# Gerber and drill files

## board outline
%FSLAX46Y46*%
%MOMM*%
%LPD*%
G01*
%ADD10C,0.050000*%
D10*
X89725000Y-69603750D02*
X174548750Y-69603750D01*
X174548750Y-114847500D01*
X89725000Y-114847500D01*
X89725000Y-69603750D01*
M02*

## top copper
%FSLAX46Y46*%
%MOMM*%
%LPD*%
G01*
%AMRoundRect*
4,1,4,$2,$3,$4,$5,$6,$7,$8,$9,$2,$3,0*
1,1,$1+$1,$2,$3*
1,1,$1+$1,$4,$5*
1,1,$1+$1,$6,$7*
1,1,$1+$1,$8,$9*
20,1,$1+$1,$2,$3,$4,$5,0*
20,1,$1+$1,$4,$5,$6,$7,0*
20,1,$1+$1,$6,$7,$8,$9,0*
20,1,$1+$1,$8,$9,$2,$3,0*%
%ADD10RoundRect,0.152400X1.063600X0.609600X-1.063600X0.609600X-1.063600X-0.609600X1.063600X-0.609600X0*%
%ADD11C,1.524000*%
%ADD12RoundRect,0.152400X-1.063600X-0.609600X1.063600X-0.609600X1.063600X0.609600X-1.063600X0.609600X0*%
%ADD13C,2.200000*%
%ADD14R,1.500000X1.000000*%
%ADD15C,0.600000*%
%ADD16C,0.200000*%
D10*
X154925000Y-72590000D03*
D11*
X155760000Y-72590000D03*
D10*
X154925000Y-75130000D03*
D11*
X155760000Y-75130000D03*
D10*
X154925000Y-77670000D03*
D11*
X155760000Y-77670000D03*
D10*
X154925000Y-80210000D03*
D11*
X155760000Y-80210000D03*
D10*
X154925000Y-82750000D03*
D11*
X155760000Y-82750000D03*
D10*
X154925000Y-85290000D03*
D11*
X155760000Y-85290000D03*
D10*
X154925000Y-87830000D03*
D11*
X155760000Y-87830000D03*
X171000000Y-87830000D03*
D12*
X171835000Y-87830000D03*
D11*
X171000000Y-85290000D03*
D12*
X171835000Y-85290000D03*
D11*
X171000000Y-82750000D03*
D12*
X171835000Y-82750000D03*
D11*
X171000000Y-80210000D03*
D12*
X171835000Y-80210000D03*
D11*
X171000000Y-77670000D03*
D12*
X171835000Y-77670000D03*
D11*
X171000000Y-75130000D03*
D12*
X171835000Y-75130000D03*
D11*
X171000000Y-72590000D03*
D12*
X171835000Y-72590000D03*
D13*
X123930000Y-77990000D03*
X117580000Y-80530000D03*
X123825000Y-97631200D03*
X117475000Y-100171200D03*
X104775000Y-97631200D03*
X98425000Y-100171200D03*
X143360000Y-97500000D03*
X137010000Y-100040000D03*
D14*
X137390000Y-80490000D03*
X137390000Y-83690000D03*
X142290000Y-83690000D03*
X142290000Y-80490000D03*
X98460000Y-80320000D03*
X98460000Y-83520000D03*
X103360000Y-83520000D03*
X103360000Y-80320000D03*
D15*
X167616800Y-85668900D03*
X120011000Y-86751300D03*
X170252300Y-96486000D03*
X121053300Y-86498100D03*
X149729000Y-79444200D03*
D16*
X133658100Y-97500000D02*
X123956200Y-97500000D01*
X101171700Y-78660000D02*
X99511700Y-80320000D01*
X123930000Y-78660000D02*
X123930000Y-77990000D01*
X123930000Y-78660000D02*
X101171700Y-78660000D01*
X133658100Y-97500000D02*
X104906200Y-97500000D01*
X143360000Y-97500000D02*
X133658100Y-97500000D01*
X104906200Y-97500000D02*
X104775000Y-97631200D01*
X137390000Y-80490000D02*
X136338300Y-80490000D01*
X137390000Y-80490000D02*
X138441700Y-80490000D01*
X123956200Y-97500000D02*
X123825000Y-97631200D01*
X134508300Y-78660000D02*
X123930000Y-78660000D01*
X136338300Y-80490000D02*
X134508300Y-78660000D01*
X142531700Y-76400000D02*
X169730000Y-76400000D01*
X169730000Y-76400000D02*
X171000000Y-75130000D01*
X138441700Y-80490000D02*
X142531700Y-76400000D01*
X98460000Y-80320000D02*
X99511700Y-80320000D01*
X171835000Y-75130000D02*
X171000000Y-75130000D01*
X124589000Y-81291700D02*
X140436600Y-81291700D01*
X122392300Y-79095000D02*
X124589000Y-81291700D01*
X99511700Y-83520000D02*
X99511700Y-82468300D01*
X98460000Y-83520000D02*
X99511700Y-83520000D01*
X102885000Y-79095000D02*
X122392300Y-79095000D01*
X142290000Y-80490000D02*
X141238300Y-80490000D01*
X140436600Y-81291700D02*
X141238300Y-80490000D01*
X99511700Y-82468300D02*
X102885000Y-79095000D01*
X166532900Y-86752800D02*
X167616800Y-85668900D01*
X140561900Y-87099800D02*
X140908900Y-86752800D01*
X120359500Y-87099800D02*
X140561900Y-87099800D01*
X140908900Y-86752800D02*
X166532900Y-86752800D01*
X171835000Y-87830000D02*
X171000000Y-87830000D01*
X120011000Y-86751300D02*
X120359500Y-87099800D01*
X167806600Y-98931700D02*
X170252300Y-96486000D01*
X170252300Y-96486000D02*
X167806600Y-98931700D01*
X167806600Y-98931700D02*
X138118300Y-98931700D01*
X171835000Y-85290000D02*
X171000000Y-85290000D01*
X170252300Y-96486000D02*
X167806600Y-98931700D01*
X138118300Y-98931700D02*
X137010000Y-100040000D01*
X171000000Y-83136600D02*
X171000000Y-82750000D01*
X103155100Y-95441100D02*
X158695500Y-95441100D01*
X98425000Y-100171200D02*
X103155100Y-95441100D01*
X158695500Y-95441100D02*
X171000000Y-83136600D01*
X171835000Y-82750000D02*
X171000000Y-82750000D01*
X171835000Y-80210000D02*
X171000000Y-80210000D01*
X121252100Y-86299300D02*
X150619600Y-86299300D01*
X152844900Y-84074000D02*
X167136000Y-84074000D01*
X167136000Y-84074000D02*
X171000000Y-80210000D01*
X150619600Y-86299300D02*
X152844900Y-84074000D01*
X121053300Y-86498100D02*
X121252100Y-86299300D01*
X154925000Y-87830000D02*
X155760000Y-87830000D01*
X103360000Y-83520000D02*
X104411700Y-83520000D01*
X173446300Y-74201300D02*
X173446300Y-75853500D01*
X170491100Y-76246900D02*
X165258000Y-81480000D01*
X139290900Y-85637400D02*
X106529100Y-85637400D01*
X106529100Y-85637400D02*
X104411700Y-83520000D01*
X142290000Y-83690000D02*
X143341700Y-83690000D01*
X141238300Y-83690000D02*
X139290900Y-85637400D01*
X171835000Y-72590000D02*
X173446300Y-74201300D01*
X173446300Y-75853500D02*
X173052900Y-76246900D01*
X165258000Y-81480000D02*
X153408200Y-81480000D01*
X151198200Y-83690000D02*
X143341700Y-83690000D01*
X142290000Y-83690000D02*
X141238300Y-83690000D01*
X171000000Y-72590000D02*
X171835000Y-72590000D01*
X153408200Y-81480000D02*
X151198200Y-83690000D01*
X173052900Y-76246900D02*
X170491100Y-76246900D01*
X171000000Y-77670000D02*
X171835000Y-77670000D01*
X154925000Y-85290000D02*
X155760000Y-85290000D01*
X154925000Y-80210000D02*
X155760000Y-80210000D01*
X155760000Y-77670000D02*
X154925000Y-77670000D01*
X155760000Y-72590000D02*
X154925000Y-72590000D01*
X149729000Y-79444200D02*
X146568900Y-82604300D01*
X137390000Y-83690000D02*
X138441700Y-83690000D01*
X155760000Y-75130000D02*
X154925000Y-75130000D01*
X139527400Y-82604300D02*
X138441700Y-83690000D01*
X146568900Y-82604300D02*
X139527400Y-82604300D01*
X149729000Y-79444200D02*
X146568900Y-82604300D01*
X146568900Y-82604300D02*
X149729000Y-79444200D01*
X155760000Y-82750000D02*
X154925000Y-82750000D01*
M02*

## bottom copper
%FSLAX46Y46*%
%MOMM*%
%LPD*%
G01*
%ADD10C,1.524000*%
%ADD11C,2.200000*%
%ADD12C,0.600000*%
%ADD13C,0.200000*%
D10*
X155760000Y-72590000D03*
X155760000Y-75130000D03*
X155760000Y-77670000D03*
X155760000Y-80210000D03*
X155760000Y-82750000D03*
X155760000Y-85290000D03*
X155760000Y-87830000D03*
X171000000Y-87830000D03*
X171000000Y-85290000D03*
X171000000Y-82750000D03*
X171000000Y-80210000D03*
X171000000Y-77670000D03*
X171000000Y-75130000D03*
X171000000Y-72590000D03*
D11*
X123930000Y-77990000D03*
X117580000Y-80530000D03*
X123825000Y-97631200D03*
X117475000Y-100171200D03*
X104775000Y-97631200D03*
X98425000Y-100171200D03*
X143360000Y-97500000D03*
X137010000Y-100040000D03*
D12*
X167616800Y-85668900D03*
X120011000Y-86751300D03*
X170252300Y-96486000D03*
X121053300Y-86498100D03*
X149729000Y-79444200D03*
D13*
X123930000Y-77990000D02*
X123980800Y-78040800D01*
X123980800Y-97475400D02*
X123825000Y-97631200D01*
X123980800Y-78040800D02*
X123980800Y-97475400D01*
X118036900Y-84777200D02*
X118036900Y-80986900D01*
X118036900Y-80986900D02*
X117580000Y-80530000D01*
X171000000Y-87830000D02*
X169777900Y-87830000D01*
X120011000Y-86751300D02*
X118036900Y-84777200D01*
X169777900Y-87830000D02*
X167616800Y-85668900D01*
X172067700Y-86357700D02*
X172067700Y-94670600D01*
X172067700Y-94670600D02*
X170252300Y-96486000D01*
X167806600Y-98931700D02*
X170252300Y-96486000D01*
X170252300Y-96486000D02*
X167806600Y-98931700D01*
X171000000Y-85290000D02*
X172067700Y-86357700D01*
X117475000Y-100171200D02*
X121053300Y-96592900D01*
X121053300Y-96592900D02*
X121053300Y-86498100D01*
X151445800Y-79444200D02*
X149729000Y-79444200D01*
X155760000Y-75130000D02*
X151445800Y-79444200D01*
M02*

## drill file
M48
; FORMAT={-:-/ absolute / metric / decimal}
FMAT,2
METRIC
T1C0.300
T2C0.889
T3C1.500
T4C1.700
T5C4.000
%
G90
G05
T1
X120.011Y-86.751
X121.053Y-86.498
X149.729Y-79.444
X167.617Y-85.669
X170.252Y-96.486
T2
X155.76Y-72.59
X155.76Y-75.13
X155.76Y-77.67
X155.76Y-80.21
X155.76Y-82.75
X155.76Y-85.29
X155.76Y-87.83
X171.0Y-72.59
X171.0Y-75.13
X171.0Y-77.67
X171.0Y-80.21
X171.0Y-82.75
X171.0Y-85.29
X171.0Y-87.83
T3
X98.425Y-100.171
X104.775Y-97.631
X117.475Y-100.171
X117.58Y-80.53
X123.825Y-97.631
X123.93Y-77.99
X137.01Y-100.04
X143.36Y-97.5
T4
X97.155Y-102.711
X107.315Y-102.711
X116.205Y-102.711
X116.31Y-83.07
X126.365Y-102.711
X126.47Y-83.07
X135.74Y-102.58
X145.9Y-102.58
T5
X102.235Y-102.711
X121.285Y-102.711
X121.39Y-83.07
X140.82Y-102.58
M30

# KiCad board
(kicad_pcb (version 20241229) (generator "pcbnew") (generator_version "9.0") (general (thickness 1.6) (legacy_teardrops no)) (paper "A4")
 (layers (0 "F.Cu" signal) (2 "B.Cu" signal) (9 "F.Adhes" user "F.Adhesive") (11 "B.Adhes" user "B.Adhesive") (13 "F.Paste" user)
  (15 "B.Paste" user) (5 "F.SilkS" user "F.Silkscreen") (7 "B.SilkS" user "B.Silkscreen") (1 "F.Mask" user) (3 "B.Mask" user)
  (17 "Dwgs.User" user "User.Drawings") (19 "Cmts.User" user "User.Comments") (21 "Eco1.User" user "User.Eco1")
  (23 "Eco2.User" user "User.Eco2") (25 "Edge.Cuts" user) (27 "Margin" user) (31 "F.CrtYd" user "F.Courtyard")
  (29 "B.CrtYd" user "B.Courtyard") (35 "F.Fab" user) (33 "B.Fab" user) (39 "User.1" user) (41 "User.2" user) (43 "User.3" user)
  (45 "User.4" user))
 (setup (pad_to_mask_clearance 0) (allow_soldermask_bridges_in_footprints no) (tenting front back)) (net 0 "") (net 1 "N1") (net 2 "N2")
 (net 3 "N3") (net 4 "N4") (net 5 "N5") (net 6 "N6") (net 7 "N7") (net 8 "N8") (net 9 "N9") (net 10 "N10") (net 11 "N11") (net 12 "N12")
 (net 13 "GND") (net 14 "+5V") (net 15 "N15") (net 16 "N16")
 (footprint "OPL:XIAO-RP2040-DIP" (layer "F.Cu") (at 163.38 80.21)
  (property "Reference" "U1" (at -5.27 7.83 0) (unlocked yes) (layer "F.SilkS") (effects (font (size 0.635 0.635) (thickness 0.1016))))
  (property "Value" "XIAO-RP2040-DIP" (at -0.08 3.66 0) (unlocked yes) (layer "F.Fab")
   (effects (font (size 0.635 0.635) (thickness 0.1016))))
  (pad "1" smd roundrect (at -8.455 -7.62 180) (size 2.432 1.524) (layers "F.Cu" "F.Mask") (roundrect_rratio 0.1) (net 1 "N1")
   (thermal_bridge_angle 45))
  (pad "1" thru_hole circle (at -7.62 -7.62 180) (size 1.524 1.524) (drill 0.889) (layers "*.Cu" "*.Mask") (remove_unused_layers no)
   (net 1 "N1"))
  (pad "2" smd roundrect (at -8.455 -5.08 180) (size 2.432 1.524) (layers "F.Cu" "F.Mask") (roundrect_rratio 0.1) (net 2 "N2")
   (thermal_bridge_angle 45))
  (pad "2" thru_hole circle (at -7.62 -5.08 180) (size 1.524 1.524) (drill 0.889) (layers "*.Cu" "*.Mask") (remove_unused_layers no)
   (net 2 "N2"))
  (pad "3" smd roundrect (at -8.455 -2.54 180) (size 2.432 1.524) (layers "F.Cu" "F.Mask") (roundrect_rratio 0.1) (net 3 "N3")
   (thermal_bridge_angle 45))
  (pad "3" thru_hole circle (at -7.62 -2.54 180) (size 1.524 1.524) (drill 0.889) (layers "*.Cu" "*.Mask") (remove_unused_layers no)
   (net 3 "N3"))
  (pad "4" smd roundrect (at -8.455 0 180) (size 2.432 1.524) (layers "F.Cu" "F.Mask") (roundrect_rratio 0.1) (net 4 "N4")
   (thermal_bridge_angle 45))
  (pad "4" thru_hole circle (at -7.62 0 180) (size 1.524 1.524) (drill 0.889) (layers "*.Cu" "*.Mask") (remove_unused_layers no)
   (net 4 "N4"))
  (pad "5" smd roundrect (at -8.455 2.54 180) (size 2.432 1.524) (layers "F.Cu" "F.Mask") (roundrect_rratio 0.1) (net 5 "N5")
   (thermal_bridge_angle 45))
  (pad "5" thru_hole circle (at -7.62 2.54 180) (size 1.524 1.524) (drill 0.889) (layers "*.Cu" "*.Mask") (remove_unused_layers no)
   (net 5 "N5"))
  (pad "6" smd roundrect (at -8.455 5.08 180) (size 2.432 1.524) (layers "F.Cu" "F.Mask") (roundrect_rratio 0.1) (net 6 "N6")
   (thermal_bridge_angle 45))
  (pad "6" thru_hole circle (at -7.62 5.08 180) (size 1.524 1.524) (drill 0.889) (layers "*.Cu" "*.Mask") (remove_unused_layers no)
   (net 6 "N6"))
  (pad "7" smd roundrect (at -8.455 7.62 180) (size 2.432 1.524) (layers "F.Cu" "F.Mask") (roundrect_rratio 0.1) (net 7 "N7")
   (thermal_bridge_angle 45))
  (pad "7" thru_hole circle (at -7.62 7.62 180) (size 1.524 1.524) (drill 0.889) (layers "*.Cu" "*.Mask") (remove_unused_layers no)
   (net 7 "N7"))
  (pad "8" thru_hole circle (at 7.62 7.62) (size 1.524 1.524) (drill 0.889) (layers "*.Cu" "*.Mask") (remove_unused_layers no) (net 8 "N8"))
  (pad "8" smd roundrect (at 8.455 7.62) (size 2.432 1.524) (layers "F.Cu" "F.Mask") (roundrect_rratio 0.1) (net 8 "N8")
   (thermal_bridge_angle 45))
  (pad "9" thru_hole circle (at 7.62 5.08) (size 1.524 1.524) (drill 0.889) (layers "*.Cu" "*.Mask") (remove_unused_layers no) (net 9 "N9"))
  (pad "9" smd roundrect (at 8.455 5.08) (size 2.432 1.524) (layers "F.Cu" "F.Mask") (roundrect_rratio 0.1) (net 9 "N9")
   (thermal_bridge_angle 45))
  (pad "10" thru_hole circle (at 7.62 2.54) (size 1.524 1.524) (drill 0.889) (layers "*.Cu" "*.Mask") (remove_unused_layers no)
   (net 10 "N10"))
  (pad "10" smd roundrect (at 8.455 2.54) (size 2.432 1.524) (layers "F.Cu" "F.Mask") (roundrect_rratio 0.1) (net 10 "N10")
   (thermal_bridge_angle 45))
  (pad "11" thru_hole circle (at 7.62 0) (size 1.524 1.524) (drill 0.889) (layers "*.Cu" "*.Mask") (remove_unused_layers no) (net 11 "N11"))
  (pad "11" smd roundrect (at 8.455 0) (size 2.432 1.524) (layers "F.Cu" "F.Mask") (roundrect_rratio 0.1) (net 11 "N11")
   (thermal_bridge_angle 45))
  (pad "12" thru_hole circle (at 7.62 -2.54) (size 1.524 1.524) (drill 0.889) (layers "*.Cu" "*.Mask") (remove_unused_layers no)
   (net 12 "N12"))
  (pad "12" smd roundrect (at 8.455 -2.54) (size 2.432 1.524) (layers "F.Cu" "F.Mask") (roundrect_rratio 0.1) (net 12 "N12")
   (thermal_bridge_angle 45))
  (pad "13" thru_hole circle (at 7.62 -5.08) (size 1.524 1.524) (drill 0.889) (layers "*.Cu" "*.Mask") (remove_unused_layers no)
   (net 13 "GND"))
  (pad "13" smd roundrect (at 8.455 -5.08) (size 2.432 1.524) (layers "F.Cu" "F.Mask") (roundrect_rratio 0.1) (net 13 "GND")
   (thermal_bridge_angle 45))
  (pad "14" thru_hole circle (at 7.62 -7.62) (size 1.524 1.524) (drill 0.889) (layers "*.Cu" "*.Mask") (remove_unused_layers no)
   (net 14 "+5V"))
  (pad "14" smd roundrect (at 8.455 -7.62) (size 2.432 1.524) (layers "F.Cu" "F.Mask") (roundrect_rratio 0.1) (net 14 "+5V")
   (thermal_bridge_angle 45)))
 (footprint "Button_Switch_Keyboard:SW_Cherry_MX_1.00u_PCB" (layer "F.Cu") (at 123.93 77.99)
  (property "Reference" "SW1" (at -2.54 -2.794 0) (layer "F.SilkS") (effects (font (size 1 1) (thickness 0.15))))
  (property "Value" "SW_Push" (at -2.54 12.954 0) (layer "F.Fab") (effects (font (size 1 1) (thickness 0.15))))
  (pad "" np_thru_hole circle (at -7.62 5.08) (size 1.7 1.7) (drill 1.7) (layers "*.Cu" "*.Mask"))
  (pad "" np_thru_hole circle (at -2.54 5.08) (size 4 4) (drill 4) (layers "*.Cu" "*.Mask"))
  (pad "" np_thru_hole circle (at 2.54 5.08) (size 1.7 1.7) (drill 1.7) (layers "*.Cu" "*.Mask"))
  (pad "1" thru_hole circle (at 0 0) (size 2.2 2.2) (drill 1.5) (layers "*.Cu" "*.Mask") (remove_unused_layers no) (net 13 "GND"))
  (pad "2" thru_hole circle (at -6.35 2.54) (size 2.2 2.2) (drill 1.5) (layers "*.Cu" "*.Mask") (remove_unused_layers no) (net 8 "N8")))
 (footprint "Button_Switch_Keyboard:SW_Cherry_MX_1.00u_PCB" (layer "F.Cu") (at 123.825 97.6312)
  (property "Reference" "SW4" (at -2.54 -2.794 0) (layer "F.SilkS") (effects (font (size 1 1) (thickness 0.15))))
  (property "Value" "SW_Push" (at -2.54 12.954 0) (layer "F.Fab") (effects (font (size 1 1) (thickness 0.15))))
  (pad "" np_thru_hole circle (at -7.62 5.08) (size 1.7 1.7) (drill 1.7) (layers "*.Cu" "*.Mask"))
  (pad "" np_thru_hole circle (at -2.54 5.08) (size 4 4) (drill 4) (layers "*.Cu" "*.Mask"))
  (pad "" np_thru_hole circle (at 2.54 5.08) (size 1.7 1.7) (drill 1.7) (layers "*.Cu" "*.Mask"))
  (pad "1" thru_hole circle (at 0 0) (size 2.2 2.2) (drill 1.5) (layers "*.Cu" "*.Mask") (remove_unused_layers no) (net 13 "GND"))
  (pad "2" thru_hole circle (at -6.35 2.54) (size 2.2 2.2) (drill 1.5) (layers "*.Cu" "*.Mask") (remove_unused_layers no) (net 11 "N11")))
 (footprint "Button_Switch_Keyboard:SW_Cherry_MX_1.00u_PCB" (layer "F.Cu") (at 104.775 97.6312)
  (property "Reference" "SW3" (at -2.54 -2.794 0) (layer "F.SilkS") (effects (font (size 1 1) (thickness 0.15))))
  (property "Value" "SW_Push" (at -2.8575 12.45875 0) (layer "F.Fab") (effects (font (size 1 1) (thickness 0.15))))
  (pad "" np_thru_hole circle (at -7.62 5.08) (size 1.7 1.7) (drill 1.7) (layers "*.Cu" "*.Mask"))
  (pad "" np_thru_hole circle (at -2.54 5.08) (size 4 4) (drill 4) (layers "*.Cu" "*.Mask"))
  (pad "" np_thru_hole circle (at 2.54 5.08) (size 1.7 1.7) (drill 1.7) (layers "*.Cu" "*.Mask"))
  (pad "1" thru_hole circle (at 0 0) (size 2.2 2.2) (drill 1.5) (layers "*.Cu" "*.Mask") (remove_unused_layers no) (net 13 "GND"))
  (pad "2" thru_hole circle (at -6.35 2.54) (size 2.2 2.2) (drill 1.5) (layers "*.Cu" "*.Mask") (remove_unused_layers no) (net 10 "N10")))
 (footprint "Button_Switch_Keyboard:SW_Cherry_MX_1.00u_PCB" (layer "F.Cu") (at 143.36 97.5)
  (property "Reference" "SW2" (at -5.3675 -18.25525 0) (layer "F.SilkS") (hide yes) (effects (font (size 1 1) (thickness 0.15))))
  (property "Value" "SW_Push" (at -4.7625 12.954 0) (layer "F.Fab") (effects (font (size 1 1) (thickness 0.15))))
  (pad "" np_thru_hole circle (at -7.62 5.08) (size 1.7 1.7) (drill 1.7) (layers "*.Cu" "*.Mask"))
  (pad "" np_thru_hole circle (at -2.54 5.08) (size 4 4) (drill 4) (layers "*.Cu" "*.Mask"))
  (pad "" np_thru_hole circle (at 2.54 5.08) (size 1.7 1.7) (drill 1.7) (layers "*.Cu" "*.Mask"))
  (pad "1" thru_hole circle (at 0 0) (size 2.2 2.2) (drill 1.5) (layers "*.Cu" "*.Mask") (remove_unused_layers no) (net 13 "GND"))
  (pad "2" thru_hole circle (at -6.35 2.54) (size 2.2 2.2) (drill 1.5) (layers "*.Cu" "*.Mask") (remove_unused_layers no) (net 9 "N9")))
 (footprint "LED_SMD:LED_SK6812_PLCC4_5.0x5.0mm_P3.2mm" (layer "F.Cu") (at 139.84 82.09)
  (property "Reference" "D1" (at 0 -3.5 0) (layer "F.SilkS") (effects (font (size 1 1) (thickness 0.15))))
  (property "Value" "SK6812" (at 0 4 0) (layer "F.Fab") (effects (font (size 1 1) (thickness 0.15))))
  (pad "1" smd rect (at -2.45 -1.6 180) (size 1.5 1) (layers "F.Cu" "F.Mask" "F.Paste") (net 13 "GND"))
  (pad "2" smd rect (at -2.45 1.6 180) (size 1.5 1) (layers "F.Cu" "F.Mask" "F.Paste") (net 2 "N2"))
  (pad "3" smd rect (at 2.45 1.6 180) (size 1.5 1) (layers "F.Cu" "F.Mask" "F.Paste") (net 14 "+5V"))
  (pad "4" smd rect (at 2.45 -1.6 180) (size 1.5 1) (layers "F.Cu" "F.Mask" "F.Paste") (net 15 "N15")))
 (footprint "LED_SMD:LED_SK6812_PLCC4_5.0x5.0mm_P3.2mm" (layer "F.Cu") (at 100.91 81.92)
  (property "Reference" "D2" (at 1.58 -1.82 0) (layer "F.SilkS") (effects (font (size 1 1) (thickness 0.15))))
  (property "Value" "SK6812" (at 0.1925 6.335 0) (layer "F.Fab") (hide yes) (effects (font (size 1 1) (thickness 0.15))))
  (pad "1" smd rect (at -2.45 -1.6 180) (size 1.5 1) (layers "F.Cu" "F.Mask" "F.Paste") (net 13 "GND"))
  (pad "2" smd rect (at -2.45 1.6 180) (size 1.5 1) (layers "F.Cu" "F.Mask" "F.Paste") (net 15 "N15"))
  (pad "3" smd rect (at 2.45 1.6 180) (size 1.5 1) (layers "F.Cu" "F.Mask" "F.Paste") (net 14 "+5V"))
  (pad "4" smd rect (at 2.45 -1.6 180) (size 1.5 1) (layers "F.Cu" "F.Mask" "F.Paste") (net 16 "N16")))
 (gr_rect (start 89.725 69.60375) (end 174.54875 114.8475) (stroke (width 0.05) (type default)) (fill no) (layer "Edge.Cuts"))
 (segment (start 133.6581 97.5) (end 123.9562 97.5) (width 0.2) (layer "F.Cu") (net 13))
 (segment (start 101.1717 78.66) (end 99.5117 80.32) (width 0.2) (layer "F.Cu") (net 13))
 (segment (start 123.93 78.66) (end 123.93 77.99) (width 0.2) (layer "F.Cu") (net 13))
 (segment (start 123.93 78.66) (end 101.1717 78.66) (width 0.2) (layer "F.Cu") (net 13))
 (segment (start 133.6581 97.5) (end 104.9062 97.5) (width 0.2) (layer "F.Cu") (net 13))
 (segment (start 143.36 97.5) (end 133.6581 97.5) (width 0.2) (layer "F.Cu") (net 13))
 (segment (start 104.9062 97.5) (end 104.775 97.6312) (width 0.2) (layer "F.Cu") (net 13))
 (segment (start 137.39 80.49) (end 136.3383 80.49) (width 0.2) (layer "F.Cu") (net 13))
 (segment (start 137.39 80.49) (end 138.4417 80.49) (width 0.2) (layer "F.Cu") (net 13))
 (segment (start 123.9562 97.5) (end 123.825 97.6312) (width 0.2) (layer "F.Cu") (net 13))
 (segment (start 134.5083 78.66) (end 123.93 78.66) (width 0.2) (layer "F.Cu") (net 13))
 (segment (start 136.3383 80.49) (end 134.5083 78.66) (width 0.2) (layer "F.Cu") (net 13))
 (segment (start 142.5317 76.4) (end 169.73 76.4) (width 0.2) (layer "F.Cu") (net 13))
 (segment (start 169.73 76.4) (end 171 75.13) (width 0.2) (layer "F.Cu") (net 13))
 (segment (start 138.4417 80.49) (end 142.5317 76.4) (width 0.2) (layer "F.Cu") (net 13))
 (segment (start 98.46 80.32) (end 99.5117 80.32) (width 0.2) (layer "F.Cu") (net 13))
 (segment (start 171.835 75.13) (end 171 75.13) (width 0.2) (layer "F.Cu") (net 13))
 (segment (start 123.93 77.99) (end 123.9808 78.0408) (width 0.2) (layer "B.Cu") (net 13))
 (segment (start 123.9808 97.4754) (end 123.825 97.6312) (width 0.2) (layer "B.Cu") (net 13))
 (segment (start 123.9808 78.0408) (end 123.9808 97.4754) (width 0.2) (layer "B.Cu") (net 13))
 (segment (start 124.589 81.2917) (end 140.4366 81.2917) (width 0.2) (layer "F.Cu") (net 15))
 (segment (start 122.3923 79.095) (end 124.589 81.2917) (width 0.2) (layer "F.Cu") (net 15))
 (segment (start 99.5117 83.52) (end 99.5117 82.4683) (width 0.2) (layer "F.Cu") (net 15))
 (segment (start 98.46 83.52) (end 99.5117 83.52) (width 0.2) (layer "F.Cu") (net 15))
 (segment (start 102.885 79.095) (end 122.3923 79.095) (width 0.2) (layer "F.Cu") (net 15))
 (segment (start 142.29 80.49) (end 141.2383 80.49) (width 0.2) (layer "F.Cu") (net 15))
 (segment (start 140.4366 81.2917) (end 141.2383 80.49) (width 0.2) (layer "F.Cu") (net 15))
 (segment (start 99.5117 82.4683) (end 102.885 79.095) (width 0.2) (layer "F.Cu") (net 15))
 (segment (start 166.5329 86.7528) (end 167.6168 85.6689) (width 0.2) (layer "F.Cu") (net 8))
 (segment (start 140.5619 87.0998) (end 140.9089 86.7528) (width 0.2) (layer "F.Cu") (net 8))
 (segment (start 120.3595 87.0998) (end 140.5619 87.0998) (width 0.2) (layer "F.Cu") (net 8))
 (segment (start 140.9089 86.7528) (end 166.5329 86.7528) (width 0.2) (layer "F.Cu") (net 8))
 (segment (start 171.835 87.83) (end 171 87.83) (width 0.2) (layer "F.Cu") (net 8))
 (segment (start 120.011 86.7513) (end 120.3595 87.0998) (width 0.2) (layer "F.Cu") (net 8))
 (via (at 167.6168 85.6689) (size 0.6) (drill 0.3) (layers "F.Cu" "B.Cu") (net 8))
 (via (at 120.011 86.7513) (size 0.6) (drill 0.3) (layers "F.Cu" "B.Cu") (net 8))
 (segment (start 118.0369 84.7772) (end 118.0369 80.9869) (width 0.2) (layer "B.Cu") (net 8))
 (segment (start 118.0369 80.9869) (end 117.58 80.53) (width 0.2) (layer "B.Cu") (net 8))
 (segment (start 171 87.83) (end 169.7779 87.83) (width 0.2) (layer "B.Cu") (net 8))
 (segment (start 120.011 86.7513) (end 118.0369 84.7772) (width 0.2) (layer "B.Cu") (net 8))
 (segment (start 169.7779 87.83) (end 167.6168 85.6689) (width 0.2) (layer "B.Cu") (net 8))
 (segment (start 167.8066 98.9317) (end 170.2523 96.486) (width 0.2) (layer "F.Cu") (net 9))
 (segment (start 170.2523 96.486) (end 167.8066 98.9317) (width 0.2) (layer "F.Cu") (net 9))
 (segment (start 167.8066 98.9317) (end 138.1183 98.9317) (width 0.2) (layer "F.Cu") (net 9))
 (segment (start 171.835 85.29) (end 171 85.29) (width 0.2) (layer "F.Cu") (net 9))
 (segment (start 170.2523 96.486) (end 167.8066 98.9317) (width 0.2) (layer "F.Cu") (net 9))
 (segment (start 138.1183 98.9317) (end 137.01 100.04) (width 0.2) (layer "F.Cu") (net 9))
 (via (at 170.2523 96.486) (size 0.6) (drill 0.3) (layers "F.Cu" "B.Cu") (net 9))
 (segment (start 172.0677 86.3577) (end 172.0677 94.6706) (width 0.2) (layer "B.Cu") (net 9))
 (segment (start 172.0677 94.6706) (end 170.2523 96.486) (width 0.2) (layer "B.Cu") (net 9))
 (segment (start 167.8066 98.9317) (end 170.2523 96.486) (width 0.2) (layer "B.Cu") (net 9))
 (segment (start 170.2523 96.486) (end 167.8066 98.9317) (width 0.2) (layer "B.Cu") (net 9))
 (segment (start 171 85.29) (end 172.0677 86.3577) (width 0.2) (layer "B.Cu") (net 9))
 (segment (start 171 83.1366) (end 171 82.75) (width 0.2) (layer "F.Cu") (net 10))
 (segment (start 103.1551 95.4411) (end 158.6955 95.4411) (width 0.2) (layer "F.Cu") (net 10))
 (segment (start 98.425 100.1712) (end 103.1551 95.4411) (width 0.2) (layer "F.Cu") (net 10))
 (segment (start 158.6955 95.4411) (end 171 83.1366) (width 0.2) (layer "F.Cu") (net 10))
 (segment (start 171.835 82.75) (end 171 82.75) (width 0.2) (layer "F.Cu") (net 10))
 (segment (start 171.835 80.21) (end 171 80.21) (width 0.2) (layer "F.Cu") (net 11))
 (segment (start 121.2521 86.2993) (end 150.6196 86.2993) (width 0.2) (layer "F.Cu") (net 11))
 (segment (start 152.8449 84.074) (end 167.136 84.074) (width 0.2) (layer "F.Cu") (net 11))
 (segment (start 167.136 84.074) (end 171 80.21) (width 0.2) (layer "F.Cu") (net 11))
 (segment (start 150.6196 86.2993) (end 152.8449 84.074) (width 0.2) (layer "F.Cu") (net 11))
 (segment (start 121.0533 86.4981) (end 121.2521 86.2993) (width 0.2) (layer "F.Cu") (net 11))
 (via (at 121.0533 86.4981) (size 0.6) (drill 0.3) (layers "F.Cu" "B.Cu") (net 11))
 (segment (start 117.475 100.1712) (end 121.0533 96.5929) (width 0.2) (layer "B.Cu") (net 11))
 (segment (start 121.0533 96.5929) (end 121.0533 86.4981) (width 0.2) (layer "B.Cu") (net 11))
 (segment (start 154.925 87.83) (end 155.76 87.83) (width 0.2) (layer "F.Cu") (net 7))
 (segment (start 103.36 83.52) (end 104.4117 83.52) (width 0.2) (layer "F.Cu") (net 14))
 (segment (start 173.4463 74.2013) (end 173.4463 75.8535) (width 0.2) (layer "F.Cu") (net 14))
 (segment (start 170.4911 76.2469) (end 165.258 81.48) (width 0.2) (layer "F.Cu") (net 14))
 (segment (start 139.2909 85.6374) (end 106.5291 85.6374) (width 0.2) (layer "F.Cu") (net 14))
 (segment (start 106.5291 85.6374) (end 104.4117 83.52) (width 0.2) (layer "F.Cu") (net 14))
 (segment (start 142.29 83.69) (end 143.3417 83.69) (width 0.2) (layer "F.Cu") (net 14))
 (segment (start 141.2383 83.69) (end 139.2909 85.6374) (width 0.2) (layer "F.Cu") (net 14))
 (segment (start 171.835 72.59) (end 173.4463 74.2013) (width 0.2) (layer "F.Cu") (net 14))
 (segment (start 173.4463 75.8535) (end 173.0529 76.2469) (width 0.2) (layer "F.Cu") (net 14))
 (segment (start 165.258 81.48) (end 153.4082 81.48) (width 0.2) (layer "F.Cu") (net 14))
 (segment (start 151.1982 83.69) (end 143.3417 83.69) (width 0.2) (layer "F.Cu") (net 14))
 (segment (start 142.29 83.69) (end 141.2383 83.69) (width 0.2) (layer "F.Cu") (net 14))
 (segment (start 171 72.59) (end 171.835 72.59) (width 0.2) (layer "F.Cu") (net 14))
 (segment (start 153.4082 81.48) (end 151.1982 83.69) (width 0.2) (layer "F.Cu") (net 14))
 (segment (start 173.0529 76.2469) (end 170.4911 76.2469) (width 0.2) (layer "F.Cu") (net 14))
 (segment (start 171 77.67) (end 171.835 77.67) (width 0.2) (layer "F.Cu") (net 12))
 (segment (start 154.925 85.29) (end 155.76 85.29) (width 0.2) (layer "F.Cu") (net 6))
 (segment (start 154.925 80.21) (end 155.76 80.21) (width 0.2) (layer "F.Cu") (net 4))
 (segment (start 155.76 77.67) (end 154.925 77.67) (width 0.2) (layer "F.Cu") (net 3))
 (segment (start 155.76 72.59) (end 154.925 72.59) (width 0.2) (layer "F.Cu") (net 1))
 (segment (start 149.729 79.4442) (end 146.5689 82.6043) (width 0.2) (layer "F.Cu") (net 2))
 (segment (start 137.39 83.69) (end 138.4417 83.69) (width 0.2) (layer "F.Cu") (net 2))
 (segment (start 155.76 75.13) (end 154.925 75.13) (width 0.2) (layer "F.Cu") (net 2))
 (segment (start 139.5274 82.6043) (end 138.4417 83.69) (width 0.2) (layer "F.Cu") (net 2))
 (segment (start 146.5689 82.6043) (end 139.5274 82.6043) (width 0.2) (layer "F.Cu") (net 2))
 (segment (start 149.729 79.4442) (end 146.5689 82.6043) (width 0.2) (layer "F.Cu") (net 2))
 (segment (start 146.5689 82.6043) (end 149.729 79.4442) (width 0.2) (layer "F.Cu") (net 2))
 (via (at 149.729 79.4442) (size 0.6) (drill 0.3) (layers "F.Cu" "B.Cu") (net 2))
 (segment (start 151.4458 79.4442) (end 149.729 79.4442) (width 0.2) (layer "B.Cu") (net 2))
 (segment (start 155.76 75.13) (end 151.4458 79.4442) (width 0.2) (layer "B.Cu") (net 2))
 (segment (start 155.76 82.75) (end 154.925 82.75) (width 0.2) (layer "F.Cu") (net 5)))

